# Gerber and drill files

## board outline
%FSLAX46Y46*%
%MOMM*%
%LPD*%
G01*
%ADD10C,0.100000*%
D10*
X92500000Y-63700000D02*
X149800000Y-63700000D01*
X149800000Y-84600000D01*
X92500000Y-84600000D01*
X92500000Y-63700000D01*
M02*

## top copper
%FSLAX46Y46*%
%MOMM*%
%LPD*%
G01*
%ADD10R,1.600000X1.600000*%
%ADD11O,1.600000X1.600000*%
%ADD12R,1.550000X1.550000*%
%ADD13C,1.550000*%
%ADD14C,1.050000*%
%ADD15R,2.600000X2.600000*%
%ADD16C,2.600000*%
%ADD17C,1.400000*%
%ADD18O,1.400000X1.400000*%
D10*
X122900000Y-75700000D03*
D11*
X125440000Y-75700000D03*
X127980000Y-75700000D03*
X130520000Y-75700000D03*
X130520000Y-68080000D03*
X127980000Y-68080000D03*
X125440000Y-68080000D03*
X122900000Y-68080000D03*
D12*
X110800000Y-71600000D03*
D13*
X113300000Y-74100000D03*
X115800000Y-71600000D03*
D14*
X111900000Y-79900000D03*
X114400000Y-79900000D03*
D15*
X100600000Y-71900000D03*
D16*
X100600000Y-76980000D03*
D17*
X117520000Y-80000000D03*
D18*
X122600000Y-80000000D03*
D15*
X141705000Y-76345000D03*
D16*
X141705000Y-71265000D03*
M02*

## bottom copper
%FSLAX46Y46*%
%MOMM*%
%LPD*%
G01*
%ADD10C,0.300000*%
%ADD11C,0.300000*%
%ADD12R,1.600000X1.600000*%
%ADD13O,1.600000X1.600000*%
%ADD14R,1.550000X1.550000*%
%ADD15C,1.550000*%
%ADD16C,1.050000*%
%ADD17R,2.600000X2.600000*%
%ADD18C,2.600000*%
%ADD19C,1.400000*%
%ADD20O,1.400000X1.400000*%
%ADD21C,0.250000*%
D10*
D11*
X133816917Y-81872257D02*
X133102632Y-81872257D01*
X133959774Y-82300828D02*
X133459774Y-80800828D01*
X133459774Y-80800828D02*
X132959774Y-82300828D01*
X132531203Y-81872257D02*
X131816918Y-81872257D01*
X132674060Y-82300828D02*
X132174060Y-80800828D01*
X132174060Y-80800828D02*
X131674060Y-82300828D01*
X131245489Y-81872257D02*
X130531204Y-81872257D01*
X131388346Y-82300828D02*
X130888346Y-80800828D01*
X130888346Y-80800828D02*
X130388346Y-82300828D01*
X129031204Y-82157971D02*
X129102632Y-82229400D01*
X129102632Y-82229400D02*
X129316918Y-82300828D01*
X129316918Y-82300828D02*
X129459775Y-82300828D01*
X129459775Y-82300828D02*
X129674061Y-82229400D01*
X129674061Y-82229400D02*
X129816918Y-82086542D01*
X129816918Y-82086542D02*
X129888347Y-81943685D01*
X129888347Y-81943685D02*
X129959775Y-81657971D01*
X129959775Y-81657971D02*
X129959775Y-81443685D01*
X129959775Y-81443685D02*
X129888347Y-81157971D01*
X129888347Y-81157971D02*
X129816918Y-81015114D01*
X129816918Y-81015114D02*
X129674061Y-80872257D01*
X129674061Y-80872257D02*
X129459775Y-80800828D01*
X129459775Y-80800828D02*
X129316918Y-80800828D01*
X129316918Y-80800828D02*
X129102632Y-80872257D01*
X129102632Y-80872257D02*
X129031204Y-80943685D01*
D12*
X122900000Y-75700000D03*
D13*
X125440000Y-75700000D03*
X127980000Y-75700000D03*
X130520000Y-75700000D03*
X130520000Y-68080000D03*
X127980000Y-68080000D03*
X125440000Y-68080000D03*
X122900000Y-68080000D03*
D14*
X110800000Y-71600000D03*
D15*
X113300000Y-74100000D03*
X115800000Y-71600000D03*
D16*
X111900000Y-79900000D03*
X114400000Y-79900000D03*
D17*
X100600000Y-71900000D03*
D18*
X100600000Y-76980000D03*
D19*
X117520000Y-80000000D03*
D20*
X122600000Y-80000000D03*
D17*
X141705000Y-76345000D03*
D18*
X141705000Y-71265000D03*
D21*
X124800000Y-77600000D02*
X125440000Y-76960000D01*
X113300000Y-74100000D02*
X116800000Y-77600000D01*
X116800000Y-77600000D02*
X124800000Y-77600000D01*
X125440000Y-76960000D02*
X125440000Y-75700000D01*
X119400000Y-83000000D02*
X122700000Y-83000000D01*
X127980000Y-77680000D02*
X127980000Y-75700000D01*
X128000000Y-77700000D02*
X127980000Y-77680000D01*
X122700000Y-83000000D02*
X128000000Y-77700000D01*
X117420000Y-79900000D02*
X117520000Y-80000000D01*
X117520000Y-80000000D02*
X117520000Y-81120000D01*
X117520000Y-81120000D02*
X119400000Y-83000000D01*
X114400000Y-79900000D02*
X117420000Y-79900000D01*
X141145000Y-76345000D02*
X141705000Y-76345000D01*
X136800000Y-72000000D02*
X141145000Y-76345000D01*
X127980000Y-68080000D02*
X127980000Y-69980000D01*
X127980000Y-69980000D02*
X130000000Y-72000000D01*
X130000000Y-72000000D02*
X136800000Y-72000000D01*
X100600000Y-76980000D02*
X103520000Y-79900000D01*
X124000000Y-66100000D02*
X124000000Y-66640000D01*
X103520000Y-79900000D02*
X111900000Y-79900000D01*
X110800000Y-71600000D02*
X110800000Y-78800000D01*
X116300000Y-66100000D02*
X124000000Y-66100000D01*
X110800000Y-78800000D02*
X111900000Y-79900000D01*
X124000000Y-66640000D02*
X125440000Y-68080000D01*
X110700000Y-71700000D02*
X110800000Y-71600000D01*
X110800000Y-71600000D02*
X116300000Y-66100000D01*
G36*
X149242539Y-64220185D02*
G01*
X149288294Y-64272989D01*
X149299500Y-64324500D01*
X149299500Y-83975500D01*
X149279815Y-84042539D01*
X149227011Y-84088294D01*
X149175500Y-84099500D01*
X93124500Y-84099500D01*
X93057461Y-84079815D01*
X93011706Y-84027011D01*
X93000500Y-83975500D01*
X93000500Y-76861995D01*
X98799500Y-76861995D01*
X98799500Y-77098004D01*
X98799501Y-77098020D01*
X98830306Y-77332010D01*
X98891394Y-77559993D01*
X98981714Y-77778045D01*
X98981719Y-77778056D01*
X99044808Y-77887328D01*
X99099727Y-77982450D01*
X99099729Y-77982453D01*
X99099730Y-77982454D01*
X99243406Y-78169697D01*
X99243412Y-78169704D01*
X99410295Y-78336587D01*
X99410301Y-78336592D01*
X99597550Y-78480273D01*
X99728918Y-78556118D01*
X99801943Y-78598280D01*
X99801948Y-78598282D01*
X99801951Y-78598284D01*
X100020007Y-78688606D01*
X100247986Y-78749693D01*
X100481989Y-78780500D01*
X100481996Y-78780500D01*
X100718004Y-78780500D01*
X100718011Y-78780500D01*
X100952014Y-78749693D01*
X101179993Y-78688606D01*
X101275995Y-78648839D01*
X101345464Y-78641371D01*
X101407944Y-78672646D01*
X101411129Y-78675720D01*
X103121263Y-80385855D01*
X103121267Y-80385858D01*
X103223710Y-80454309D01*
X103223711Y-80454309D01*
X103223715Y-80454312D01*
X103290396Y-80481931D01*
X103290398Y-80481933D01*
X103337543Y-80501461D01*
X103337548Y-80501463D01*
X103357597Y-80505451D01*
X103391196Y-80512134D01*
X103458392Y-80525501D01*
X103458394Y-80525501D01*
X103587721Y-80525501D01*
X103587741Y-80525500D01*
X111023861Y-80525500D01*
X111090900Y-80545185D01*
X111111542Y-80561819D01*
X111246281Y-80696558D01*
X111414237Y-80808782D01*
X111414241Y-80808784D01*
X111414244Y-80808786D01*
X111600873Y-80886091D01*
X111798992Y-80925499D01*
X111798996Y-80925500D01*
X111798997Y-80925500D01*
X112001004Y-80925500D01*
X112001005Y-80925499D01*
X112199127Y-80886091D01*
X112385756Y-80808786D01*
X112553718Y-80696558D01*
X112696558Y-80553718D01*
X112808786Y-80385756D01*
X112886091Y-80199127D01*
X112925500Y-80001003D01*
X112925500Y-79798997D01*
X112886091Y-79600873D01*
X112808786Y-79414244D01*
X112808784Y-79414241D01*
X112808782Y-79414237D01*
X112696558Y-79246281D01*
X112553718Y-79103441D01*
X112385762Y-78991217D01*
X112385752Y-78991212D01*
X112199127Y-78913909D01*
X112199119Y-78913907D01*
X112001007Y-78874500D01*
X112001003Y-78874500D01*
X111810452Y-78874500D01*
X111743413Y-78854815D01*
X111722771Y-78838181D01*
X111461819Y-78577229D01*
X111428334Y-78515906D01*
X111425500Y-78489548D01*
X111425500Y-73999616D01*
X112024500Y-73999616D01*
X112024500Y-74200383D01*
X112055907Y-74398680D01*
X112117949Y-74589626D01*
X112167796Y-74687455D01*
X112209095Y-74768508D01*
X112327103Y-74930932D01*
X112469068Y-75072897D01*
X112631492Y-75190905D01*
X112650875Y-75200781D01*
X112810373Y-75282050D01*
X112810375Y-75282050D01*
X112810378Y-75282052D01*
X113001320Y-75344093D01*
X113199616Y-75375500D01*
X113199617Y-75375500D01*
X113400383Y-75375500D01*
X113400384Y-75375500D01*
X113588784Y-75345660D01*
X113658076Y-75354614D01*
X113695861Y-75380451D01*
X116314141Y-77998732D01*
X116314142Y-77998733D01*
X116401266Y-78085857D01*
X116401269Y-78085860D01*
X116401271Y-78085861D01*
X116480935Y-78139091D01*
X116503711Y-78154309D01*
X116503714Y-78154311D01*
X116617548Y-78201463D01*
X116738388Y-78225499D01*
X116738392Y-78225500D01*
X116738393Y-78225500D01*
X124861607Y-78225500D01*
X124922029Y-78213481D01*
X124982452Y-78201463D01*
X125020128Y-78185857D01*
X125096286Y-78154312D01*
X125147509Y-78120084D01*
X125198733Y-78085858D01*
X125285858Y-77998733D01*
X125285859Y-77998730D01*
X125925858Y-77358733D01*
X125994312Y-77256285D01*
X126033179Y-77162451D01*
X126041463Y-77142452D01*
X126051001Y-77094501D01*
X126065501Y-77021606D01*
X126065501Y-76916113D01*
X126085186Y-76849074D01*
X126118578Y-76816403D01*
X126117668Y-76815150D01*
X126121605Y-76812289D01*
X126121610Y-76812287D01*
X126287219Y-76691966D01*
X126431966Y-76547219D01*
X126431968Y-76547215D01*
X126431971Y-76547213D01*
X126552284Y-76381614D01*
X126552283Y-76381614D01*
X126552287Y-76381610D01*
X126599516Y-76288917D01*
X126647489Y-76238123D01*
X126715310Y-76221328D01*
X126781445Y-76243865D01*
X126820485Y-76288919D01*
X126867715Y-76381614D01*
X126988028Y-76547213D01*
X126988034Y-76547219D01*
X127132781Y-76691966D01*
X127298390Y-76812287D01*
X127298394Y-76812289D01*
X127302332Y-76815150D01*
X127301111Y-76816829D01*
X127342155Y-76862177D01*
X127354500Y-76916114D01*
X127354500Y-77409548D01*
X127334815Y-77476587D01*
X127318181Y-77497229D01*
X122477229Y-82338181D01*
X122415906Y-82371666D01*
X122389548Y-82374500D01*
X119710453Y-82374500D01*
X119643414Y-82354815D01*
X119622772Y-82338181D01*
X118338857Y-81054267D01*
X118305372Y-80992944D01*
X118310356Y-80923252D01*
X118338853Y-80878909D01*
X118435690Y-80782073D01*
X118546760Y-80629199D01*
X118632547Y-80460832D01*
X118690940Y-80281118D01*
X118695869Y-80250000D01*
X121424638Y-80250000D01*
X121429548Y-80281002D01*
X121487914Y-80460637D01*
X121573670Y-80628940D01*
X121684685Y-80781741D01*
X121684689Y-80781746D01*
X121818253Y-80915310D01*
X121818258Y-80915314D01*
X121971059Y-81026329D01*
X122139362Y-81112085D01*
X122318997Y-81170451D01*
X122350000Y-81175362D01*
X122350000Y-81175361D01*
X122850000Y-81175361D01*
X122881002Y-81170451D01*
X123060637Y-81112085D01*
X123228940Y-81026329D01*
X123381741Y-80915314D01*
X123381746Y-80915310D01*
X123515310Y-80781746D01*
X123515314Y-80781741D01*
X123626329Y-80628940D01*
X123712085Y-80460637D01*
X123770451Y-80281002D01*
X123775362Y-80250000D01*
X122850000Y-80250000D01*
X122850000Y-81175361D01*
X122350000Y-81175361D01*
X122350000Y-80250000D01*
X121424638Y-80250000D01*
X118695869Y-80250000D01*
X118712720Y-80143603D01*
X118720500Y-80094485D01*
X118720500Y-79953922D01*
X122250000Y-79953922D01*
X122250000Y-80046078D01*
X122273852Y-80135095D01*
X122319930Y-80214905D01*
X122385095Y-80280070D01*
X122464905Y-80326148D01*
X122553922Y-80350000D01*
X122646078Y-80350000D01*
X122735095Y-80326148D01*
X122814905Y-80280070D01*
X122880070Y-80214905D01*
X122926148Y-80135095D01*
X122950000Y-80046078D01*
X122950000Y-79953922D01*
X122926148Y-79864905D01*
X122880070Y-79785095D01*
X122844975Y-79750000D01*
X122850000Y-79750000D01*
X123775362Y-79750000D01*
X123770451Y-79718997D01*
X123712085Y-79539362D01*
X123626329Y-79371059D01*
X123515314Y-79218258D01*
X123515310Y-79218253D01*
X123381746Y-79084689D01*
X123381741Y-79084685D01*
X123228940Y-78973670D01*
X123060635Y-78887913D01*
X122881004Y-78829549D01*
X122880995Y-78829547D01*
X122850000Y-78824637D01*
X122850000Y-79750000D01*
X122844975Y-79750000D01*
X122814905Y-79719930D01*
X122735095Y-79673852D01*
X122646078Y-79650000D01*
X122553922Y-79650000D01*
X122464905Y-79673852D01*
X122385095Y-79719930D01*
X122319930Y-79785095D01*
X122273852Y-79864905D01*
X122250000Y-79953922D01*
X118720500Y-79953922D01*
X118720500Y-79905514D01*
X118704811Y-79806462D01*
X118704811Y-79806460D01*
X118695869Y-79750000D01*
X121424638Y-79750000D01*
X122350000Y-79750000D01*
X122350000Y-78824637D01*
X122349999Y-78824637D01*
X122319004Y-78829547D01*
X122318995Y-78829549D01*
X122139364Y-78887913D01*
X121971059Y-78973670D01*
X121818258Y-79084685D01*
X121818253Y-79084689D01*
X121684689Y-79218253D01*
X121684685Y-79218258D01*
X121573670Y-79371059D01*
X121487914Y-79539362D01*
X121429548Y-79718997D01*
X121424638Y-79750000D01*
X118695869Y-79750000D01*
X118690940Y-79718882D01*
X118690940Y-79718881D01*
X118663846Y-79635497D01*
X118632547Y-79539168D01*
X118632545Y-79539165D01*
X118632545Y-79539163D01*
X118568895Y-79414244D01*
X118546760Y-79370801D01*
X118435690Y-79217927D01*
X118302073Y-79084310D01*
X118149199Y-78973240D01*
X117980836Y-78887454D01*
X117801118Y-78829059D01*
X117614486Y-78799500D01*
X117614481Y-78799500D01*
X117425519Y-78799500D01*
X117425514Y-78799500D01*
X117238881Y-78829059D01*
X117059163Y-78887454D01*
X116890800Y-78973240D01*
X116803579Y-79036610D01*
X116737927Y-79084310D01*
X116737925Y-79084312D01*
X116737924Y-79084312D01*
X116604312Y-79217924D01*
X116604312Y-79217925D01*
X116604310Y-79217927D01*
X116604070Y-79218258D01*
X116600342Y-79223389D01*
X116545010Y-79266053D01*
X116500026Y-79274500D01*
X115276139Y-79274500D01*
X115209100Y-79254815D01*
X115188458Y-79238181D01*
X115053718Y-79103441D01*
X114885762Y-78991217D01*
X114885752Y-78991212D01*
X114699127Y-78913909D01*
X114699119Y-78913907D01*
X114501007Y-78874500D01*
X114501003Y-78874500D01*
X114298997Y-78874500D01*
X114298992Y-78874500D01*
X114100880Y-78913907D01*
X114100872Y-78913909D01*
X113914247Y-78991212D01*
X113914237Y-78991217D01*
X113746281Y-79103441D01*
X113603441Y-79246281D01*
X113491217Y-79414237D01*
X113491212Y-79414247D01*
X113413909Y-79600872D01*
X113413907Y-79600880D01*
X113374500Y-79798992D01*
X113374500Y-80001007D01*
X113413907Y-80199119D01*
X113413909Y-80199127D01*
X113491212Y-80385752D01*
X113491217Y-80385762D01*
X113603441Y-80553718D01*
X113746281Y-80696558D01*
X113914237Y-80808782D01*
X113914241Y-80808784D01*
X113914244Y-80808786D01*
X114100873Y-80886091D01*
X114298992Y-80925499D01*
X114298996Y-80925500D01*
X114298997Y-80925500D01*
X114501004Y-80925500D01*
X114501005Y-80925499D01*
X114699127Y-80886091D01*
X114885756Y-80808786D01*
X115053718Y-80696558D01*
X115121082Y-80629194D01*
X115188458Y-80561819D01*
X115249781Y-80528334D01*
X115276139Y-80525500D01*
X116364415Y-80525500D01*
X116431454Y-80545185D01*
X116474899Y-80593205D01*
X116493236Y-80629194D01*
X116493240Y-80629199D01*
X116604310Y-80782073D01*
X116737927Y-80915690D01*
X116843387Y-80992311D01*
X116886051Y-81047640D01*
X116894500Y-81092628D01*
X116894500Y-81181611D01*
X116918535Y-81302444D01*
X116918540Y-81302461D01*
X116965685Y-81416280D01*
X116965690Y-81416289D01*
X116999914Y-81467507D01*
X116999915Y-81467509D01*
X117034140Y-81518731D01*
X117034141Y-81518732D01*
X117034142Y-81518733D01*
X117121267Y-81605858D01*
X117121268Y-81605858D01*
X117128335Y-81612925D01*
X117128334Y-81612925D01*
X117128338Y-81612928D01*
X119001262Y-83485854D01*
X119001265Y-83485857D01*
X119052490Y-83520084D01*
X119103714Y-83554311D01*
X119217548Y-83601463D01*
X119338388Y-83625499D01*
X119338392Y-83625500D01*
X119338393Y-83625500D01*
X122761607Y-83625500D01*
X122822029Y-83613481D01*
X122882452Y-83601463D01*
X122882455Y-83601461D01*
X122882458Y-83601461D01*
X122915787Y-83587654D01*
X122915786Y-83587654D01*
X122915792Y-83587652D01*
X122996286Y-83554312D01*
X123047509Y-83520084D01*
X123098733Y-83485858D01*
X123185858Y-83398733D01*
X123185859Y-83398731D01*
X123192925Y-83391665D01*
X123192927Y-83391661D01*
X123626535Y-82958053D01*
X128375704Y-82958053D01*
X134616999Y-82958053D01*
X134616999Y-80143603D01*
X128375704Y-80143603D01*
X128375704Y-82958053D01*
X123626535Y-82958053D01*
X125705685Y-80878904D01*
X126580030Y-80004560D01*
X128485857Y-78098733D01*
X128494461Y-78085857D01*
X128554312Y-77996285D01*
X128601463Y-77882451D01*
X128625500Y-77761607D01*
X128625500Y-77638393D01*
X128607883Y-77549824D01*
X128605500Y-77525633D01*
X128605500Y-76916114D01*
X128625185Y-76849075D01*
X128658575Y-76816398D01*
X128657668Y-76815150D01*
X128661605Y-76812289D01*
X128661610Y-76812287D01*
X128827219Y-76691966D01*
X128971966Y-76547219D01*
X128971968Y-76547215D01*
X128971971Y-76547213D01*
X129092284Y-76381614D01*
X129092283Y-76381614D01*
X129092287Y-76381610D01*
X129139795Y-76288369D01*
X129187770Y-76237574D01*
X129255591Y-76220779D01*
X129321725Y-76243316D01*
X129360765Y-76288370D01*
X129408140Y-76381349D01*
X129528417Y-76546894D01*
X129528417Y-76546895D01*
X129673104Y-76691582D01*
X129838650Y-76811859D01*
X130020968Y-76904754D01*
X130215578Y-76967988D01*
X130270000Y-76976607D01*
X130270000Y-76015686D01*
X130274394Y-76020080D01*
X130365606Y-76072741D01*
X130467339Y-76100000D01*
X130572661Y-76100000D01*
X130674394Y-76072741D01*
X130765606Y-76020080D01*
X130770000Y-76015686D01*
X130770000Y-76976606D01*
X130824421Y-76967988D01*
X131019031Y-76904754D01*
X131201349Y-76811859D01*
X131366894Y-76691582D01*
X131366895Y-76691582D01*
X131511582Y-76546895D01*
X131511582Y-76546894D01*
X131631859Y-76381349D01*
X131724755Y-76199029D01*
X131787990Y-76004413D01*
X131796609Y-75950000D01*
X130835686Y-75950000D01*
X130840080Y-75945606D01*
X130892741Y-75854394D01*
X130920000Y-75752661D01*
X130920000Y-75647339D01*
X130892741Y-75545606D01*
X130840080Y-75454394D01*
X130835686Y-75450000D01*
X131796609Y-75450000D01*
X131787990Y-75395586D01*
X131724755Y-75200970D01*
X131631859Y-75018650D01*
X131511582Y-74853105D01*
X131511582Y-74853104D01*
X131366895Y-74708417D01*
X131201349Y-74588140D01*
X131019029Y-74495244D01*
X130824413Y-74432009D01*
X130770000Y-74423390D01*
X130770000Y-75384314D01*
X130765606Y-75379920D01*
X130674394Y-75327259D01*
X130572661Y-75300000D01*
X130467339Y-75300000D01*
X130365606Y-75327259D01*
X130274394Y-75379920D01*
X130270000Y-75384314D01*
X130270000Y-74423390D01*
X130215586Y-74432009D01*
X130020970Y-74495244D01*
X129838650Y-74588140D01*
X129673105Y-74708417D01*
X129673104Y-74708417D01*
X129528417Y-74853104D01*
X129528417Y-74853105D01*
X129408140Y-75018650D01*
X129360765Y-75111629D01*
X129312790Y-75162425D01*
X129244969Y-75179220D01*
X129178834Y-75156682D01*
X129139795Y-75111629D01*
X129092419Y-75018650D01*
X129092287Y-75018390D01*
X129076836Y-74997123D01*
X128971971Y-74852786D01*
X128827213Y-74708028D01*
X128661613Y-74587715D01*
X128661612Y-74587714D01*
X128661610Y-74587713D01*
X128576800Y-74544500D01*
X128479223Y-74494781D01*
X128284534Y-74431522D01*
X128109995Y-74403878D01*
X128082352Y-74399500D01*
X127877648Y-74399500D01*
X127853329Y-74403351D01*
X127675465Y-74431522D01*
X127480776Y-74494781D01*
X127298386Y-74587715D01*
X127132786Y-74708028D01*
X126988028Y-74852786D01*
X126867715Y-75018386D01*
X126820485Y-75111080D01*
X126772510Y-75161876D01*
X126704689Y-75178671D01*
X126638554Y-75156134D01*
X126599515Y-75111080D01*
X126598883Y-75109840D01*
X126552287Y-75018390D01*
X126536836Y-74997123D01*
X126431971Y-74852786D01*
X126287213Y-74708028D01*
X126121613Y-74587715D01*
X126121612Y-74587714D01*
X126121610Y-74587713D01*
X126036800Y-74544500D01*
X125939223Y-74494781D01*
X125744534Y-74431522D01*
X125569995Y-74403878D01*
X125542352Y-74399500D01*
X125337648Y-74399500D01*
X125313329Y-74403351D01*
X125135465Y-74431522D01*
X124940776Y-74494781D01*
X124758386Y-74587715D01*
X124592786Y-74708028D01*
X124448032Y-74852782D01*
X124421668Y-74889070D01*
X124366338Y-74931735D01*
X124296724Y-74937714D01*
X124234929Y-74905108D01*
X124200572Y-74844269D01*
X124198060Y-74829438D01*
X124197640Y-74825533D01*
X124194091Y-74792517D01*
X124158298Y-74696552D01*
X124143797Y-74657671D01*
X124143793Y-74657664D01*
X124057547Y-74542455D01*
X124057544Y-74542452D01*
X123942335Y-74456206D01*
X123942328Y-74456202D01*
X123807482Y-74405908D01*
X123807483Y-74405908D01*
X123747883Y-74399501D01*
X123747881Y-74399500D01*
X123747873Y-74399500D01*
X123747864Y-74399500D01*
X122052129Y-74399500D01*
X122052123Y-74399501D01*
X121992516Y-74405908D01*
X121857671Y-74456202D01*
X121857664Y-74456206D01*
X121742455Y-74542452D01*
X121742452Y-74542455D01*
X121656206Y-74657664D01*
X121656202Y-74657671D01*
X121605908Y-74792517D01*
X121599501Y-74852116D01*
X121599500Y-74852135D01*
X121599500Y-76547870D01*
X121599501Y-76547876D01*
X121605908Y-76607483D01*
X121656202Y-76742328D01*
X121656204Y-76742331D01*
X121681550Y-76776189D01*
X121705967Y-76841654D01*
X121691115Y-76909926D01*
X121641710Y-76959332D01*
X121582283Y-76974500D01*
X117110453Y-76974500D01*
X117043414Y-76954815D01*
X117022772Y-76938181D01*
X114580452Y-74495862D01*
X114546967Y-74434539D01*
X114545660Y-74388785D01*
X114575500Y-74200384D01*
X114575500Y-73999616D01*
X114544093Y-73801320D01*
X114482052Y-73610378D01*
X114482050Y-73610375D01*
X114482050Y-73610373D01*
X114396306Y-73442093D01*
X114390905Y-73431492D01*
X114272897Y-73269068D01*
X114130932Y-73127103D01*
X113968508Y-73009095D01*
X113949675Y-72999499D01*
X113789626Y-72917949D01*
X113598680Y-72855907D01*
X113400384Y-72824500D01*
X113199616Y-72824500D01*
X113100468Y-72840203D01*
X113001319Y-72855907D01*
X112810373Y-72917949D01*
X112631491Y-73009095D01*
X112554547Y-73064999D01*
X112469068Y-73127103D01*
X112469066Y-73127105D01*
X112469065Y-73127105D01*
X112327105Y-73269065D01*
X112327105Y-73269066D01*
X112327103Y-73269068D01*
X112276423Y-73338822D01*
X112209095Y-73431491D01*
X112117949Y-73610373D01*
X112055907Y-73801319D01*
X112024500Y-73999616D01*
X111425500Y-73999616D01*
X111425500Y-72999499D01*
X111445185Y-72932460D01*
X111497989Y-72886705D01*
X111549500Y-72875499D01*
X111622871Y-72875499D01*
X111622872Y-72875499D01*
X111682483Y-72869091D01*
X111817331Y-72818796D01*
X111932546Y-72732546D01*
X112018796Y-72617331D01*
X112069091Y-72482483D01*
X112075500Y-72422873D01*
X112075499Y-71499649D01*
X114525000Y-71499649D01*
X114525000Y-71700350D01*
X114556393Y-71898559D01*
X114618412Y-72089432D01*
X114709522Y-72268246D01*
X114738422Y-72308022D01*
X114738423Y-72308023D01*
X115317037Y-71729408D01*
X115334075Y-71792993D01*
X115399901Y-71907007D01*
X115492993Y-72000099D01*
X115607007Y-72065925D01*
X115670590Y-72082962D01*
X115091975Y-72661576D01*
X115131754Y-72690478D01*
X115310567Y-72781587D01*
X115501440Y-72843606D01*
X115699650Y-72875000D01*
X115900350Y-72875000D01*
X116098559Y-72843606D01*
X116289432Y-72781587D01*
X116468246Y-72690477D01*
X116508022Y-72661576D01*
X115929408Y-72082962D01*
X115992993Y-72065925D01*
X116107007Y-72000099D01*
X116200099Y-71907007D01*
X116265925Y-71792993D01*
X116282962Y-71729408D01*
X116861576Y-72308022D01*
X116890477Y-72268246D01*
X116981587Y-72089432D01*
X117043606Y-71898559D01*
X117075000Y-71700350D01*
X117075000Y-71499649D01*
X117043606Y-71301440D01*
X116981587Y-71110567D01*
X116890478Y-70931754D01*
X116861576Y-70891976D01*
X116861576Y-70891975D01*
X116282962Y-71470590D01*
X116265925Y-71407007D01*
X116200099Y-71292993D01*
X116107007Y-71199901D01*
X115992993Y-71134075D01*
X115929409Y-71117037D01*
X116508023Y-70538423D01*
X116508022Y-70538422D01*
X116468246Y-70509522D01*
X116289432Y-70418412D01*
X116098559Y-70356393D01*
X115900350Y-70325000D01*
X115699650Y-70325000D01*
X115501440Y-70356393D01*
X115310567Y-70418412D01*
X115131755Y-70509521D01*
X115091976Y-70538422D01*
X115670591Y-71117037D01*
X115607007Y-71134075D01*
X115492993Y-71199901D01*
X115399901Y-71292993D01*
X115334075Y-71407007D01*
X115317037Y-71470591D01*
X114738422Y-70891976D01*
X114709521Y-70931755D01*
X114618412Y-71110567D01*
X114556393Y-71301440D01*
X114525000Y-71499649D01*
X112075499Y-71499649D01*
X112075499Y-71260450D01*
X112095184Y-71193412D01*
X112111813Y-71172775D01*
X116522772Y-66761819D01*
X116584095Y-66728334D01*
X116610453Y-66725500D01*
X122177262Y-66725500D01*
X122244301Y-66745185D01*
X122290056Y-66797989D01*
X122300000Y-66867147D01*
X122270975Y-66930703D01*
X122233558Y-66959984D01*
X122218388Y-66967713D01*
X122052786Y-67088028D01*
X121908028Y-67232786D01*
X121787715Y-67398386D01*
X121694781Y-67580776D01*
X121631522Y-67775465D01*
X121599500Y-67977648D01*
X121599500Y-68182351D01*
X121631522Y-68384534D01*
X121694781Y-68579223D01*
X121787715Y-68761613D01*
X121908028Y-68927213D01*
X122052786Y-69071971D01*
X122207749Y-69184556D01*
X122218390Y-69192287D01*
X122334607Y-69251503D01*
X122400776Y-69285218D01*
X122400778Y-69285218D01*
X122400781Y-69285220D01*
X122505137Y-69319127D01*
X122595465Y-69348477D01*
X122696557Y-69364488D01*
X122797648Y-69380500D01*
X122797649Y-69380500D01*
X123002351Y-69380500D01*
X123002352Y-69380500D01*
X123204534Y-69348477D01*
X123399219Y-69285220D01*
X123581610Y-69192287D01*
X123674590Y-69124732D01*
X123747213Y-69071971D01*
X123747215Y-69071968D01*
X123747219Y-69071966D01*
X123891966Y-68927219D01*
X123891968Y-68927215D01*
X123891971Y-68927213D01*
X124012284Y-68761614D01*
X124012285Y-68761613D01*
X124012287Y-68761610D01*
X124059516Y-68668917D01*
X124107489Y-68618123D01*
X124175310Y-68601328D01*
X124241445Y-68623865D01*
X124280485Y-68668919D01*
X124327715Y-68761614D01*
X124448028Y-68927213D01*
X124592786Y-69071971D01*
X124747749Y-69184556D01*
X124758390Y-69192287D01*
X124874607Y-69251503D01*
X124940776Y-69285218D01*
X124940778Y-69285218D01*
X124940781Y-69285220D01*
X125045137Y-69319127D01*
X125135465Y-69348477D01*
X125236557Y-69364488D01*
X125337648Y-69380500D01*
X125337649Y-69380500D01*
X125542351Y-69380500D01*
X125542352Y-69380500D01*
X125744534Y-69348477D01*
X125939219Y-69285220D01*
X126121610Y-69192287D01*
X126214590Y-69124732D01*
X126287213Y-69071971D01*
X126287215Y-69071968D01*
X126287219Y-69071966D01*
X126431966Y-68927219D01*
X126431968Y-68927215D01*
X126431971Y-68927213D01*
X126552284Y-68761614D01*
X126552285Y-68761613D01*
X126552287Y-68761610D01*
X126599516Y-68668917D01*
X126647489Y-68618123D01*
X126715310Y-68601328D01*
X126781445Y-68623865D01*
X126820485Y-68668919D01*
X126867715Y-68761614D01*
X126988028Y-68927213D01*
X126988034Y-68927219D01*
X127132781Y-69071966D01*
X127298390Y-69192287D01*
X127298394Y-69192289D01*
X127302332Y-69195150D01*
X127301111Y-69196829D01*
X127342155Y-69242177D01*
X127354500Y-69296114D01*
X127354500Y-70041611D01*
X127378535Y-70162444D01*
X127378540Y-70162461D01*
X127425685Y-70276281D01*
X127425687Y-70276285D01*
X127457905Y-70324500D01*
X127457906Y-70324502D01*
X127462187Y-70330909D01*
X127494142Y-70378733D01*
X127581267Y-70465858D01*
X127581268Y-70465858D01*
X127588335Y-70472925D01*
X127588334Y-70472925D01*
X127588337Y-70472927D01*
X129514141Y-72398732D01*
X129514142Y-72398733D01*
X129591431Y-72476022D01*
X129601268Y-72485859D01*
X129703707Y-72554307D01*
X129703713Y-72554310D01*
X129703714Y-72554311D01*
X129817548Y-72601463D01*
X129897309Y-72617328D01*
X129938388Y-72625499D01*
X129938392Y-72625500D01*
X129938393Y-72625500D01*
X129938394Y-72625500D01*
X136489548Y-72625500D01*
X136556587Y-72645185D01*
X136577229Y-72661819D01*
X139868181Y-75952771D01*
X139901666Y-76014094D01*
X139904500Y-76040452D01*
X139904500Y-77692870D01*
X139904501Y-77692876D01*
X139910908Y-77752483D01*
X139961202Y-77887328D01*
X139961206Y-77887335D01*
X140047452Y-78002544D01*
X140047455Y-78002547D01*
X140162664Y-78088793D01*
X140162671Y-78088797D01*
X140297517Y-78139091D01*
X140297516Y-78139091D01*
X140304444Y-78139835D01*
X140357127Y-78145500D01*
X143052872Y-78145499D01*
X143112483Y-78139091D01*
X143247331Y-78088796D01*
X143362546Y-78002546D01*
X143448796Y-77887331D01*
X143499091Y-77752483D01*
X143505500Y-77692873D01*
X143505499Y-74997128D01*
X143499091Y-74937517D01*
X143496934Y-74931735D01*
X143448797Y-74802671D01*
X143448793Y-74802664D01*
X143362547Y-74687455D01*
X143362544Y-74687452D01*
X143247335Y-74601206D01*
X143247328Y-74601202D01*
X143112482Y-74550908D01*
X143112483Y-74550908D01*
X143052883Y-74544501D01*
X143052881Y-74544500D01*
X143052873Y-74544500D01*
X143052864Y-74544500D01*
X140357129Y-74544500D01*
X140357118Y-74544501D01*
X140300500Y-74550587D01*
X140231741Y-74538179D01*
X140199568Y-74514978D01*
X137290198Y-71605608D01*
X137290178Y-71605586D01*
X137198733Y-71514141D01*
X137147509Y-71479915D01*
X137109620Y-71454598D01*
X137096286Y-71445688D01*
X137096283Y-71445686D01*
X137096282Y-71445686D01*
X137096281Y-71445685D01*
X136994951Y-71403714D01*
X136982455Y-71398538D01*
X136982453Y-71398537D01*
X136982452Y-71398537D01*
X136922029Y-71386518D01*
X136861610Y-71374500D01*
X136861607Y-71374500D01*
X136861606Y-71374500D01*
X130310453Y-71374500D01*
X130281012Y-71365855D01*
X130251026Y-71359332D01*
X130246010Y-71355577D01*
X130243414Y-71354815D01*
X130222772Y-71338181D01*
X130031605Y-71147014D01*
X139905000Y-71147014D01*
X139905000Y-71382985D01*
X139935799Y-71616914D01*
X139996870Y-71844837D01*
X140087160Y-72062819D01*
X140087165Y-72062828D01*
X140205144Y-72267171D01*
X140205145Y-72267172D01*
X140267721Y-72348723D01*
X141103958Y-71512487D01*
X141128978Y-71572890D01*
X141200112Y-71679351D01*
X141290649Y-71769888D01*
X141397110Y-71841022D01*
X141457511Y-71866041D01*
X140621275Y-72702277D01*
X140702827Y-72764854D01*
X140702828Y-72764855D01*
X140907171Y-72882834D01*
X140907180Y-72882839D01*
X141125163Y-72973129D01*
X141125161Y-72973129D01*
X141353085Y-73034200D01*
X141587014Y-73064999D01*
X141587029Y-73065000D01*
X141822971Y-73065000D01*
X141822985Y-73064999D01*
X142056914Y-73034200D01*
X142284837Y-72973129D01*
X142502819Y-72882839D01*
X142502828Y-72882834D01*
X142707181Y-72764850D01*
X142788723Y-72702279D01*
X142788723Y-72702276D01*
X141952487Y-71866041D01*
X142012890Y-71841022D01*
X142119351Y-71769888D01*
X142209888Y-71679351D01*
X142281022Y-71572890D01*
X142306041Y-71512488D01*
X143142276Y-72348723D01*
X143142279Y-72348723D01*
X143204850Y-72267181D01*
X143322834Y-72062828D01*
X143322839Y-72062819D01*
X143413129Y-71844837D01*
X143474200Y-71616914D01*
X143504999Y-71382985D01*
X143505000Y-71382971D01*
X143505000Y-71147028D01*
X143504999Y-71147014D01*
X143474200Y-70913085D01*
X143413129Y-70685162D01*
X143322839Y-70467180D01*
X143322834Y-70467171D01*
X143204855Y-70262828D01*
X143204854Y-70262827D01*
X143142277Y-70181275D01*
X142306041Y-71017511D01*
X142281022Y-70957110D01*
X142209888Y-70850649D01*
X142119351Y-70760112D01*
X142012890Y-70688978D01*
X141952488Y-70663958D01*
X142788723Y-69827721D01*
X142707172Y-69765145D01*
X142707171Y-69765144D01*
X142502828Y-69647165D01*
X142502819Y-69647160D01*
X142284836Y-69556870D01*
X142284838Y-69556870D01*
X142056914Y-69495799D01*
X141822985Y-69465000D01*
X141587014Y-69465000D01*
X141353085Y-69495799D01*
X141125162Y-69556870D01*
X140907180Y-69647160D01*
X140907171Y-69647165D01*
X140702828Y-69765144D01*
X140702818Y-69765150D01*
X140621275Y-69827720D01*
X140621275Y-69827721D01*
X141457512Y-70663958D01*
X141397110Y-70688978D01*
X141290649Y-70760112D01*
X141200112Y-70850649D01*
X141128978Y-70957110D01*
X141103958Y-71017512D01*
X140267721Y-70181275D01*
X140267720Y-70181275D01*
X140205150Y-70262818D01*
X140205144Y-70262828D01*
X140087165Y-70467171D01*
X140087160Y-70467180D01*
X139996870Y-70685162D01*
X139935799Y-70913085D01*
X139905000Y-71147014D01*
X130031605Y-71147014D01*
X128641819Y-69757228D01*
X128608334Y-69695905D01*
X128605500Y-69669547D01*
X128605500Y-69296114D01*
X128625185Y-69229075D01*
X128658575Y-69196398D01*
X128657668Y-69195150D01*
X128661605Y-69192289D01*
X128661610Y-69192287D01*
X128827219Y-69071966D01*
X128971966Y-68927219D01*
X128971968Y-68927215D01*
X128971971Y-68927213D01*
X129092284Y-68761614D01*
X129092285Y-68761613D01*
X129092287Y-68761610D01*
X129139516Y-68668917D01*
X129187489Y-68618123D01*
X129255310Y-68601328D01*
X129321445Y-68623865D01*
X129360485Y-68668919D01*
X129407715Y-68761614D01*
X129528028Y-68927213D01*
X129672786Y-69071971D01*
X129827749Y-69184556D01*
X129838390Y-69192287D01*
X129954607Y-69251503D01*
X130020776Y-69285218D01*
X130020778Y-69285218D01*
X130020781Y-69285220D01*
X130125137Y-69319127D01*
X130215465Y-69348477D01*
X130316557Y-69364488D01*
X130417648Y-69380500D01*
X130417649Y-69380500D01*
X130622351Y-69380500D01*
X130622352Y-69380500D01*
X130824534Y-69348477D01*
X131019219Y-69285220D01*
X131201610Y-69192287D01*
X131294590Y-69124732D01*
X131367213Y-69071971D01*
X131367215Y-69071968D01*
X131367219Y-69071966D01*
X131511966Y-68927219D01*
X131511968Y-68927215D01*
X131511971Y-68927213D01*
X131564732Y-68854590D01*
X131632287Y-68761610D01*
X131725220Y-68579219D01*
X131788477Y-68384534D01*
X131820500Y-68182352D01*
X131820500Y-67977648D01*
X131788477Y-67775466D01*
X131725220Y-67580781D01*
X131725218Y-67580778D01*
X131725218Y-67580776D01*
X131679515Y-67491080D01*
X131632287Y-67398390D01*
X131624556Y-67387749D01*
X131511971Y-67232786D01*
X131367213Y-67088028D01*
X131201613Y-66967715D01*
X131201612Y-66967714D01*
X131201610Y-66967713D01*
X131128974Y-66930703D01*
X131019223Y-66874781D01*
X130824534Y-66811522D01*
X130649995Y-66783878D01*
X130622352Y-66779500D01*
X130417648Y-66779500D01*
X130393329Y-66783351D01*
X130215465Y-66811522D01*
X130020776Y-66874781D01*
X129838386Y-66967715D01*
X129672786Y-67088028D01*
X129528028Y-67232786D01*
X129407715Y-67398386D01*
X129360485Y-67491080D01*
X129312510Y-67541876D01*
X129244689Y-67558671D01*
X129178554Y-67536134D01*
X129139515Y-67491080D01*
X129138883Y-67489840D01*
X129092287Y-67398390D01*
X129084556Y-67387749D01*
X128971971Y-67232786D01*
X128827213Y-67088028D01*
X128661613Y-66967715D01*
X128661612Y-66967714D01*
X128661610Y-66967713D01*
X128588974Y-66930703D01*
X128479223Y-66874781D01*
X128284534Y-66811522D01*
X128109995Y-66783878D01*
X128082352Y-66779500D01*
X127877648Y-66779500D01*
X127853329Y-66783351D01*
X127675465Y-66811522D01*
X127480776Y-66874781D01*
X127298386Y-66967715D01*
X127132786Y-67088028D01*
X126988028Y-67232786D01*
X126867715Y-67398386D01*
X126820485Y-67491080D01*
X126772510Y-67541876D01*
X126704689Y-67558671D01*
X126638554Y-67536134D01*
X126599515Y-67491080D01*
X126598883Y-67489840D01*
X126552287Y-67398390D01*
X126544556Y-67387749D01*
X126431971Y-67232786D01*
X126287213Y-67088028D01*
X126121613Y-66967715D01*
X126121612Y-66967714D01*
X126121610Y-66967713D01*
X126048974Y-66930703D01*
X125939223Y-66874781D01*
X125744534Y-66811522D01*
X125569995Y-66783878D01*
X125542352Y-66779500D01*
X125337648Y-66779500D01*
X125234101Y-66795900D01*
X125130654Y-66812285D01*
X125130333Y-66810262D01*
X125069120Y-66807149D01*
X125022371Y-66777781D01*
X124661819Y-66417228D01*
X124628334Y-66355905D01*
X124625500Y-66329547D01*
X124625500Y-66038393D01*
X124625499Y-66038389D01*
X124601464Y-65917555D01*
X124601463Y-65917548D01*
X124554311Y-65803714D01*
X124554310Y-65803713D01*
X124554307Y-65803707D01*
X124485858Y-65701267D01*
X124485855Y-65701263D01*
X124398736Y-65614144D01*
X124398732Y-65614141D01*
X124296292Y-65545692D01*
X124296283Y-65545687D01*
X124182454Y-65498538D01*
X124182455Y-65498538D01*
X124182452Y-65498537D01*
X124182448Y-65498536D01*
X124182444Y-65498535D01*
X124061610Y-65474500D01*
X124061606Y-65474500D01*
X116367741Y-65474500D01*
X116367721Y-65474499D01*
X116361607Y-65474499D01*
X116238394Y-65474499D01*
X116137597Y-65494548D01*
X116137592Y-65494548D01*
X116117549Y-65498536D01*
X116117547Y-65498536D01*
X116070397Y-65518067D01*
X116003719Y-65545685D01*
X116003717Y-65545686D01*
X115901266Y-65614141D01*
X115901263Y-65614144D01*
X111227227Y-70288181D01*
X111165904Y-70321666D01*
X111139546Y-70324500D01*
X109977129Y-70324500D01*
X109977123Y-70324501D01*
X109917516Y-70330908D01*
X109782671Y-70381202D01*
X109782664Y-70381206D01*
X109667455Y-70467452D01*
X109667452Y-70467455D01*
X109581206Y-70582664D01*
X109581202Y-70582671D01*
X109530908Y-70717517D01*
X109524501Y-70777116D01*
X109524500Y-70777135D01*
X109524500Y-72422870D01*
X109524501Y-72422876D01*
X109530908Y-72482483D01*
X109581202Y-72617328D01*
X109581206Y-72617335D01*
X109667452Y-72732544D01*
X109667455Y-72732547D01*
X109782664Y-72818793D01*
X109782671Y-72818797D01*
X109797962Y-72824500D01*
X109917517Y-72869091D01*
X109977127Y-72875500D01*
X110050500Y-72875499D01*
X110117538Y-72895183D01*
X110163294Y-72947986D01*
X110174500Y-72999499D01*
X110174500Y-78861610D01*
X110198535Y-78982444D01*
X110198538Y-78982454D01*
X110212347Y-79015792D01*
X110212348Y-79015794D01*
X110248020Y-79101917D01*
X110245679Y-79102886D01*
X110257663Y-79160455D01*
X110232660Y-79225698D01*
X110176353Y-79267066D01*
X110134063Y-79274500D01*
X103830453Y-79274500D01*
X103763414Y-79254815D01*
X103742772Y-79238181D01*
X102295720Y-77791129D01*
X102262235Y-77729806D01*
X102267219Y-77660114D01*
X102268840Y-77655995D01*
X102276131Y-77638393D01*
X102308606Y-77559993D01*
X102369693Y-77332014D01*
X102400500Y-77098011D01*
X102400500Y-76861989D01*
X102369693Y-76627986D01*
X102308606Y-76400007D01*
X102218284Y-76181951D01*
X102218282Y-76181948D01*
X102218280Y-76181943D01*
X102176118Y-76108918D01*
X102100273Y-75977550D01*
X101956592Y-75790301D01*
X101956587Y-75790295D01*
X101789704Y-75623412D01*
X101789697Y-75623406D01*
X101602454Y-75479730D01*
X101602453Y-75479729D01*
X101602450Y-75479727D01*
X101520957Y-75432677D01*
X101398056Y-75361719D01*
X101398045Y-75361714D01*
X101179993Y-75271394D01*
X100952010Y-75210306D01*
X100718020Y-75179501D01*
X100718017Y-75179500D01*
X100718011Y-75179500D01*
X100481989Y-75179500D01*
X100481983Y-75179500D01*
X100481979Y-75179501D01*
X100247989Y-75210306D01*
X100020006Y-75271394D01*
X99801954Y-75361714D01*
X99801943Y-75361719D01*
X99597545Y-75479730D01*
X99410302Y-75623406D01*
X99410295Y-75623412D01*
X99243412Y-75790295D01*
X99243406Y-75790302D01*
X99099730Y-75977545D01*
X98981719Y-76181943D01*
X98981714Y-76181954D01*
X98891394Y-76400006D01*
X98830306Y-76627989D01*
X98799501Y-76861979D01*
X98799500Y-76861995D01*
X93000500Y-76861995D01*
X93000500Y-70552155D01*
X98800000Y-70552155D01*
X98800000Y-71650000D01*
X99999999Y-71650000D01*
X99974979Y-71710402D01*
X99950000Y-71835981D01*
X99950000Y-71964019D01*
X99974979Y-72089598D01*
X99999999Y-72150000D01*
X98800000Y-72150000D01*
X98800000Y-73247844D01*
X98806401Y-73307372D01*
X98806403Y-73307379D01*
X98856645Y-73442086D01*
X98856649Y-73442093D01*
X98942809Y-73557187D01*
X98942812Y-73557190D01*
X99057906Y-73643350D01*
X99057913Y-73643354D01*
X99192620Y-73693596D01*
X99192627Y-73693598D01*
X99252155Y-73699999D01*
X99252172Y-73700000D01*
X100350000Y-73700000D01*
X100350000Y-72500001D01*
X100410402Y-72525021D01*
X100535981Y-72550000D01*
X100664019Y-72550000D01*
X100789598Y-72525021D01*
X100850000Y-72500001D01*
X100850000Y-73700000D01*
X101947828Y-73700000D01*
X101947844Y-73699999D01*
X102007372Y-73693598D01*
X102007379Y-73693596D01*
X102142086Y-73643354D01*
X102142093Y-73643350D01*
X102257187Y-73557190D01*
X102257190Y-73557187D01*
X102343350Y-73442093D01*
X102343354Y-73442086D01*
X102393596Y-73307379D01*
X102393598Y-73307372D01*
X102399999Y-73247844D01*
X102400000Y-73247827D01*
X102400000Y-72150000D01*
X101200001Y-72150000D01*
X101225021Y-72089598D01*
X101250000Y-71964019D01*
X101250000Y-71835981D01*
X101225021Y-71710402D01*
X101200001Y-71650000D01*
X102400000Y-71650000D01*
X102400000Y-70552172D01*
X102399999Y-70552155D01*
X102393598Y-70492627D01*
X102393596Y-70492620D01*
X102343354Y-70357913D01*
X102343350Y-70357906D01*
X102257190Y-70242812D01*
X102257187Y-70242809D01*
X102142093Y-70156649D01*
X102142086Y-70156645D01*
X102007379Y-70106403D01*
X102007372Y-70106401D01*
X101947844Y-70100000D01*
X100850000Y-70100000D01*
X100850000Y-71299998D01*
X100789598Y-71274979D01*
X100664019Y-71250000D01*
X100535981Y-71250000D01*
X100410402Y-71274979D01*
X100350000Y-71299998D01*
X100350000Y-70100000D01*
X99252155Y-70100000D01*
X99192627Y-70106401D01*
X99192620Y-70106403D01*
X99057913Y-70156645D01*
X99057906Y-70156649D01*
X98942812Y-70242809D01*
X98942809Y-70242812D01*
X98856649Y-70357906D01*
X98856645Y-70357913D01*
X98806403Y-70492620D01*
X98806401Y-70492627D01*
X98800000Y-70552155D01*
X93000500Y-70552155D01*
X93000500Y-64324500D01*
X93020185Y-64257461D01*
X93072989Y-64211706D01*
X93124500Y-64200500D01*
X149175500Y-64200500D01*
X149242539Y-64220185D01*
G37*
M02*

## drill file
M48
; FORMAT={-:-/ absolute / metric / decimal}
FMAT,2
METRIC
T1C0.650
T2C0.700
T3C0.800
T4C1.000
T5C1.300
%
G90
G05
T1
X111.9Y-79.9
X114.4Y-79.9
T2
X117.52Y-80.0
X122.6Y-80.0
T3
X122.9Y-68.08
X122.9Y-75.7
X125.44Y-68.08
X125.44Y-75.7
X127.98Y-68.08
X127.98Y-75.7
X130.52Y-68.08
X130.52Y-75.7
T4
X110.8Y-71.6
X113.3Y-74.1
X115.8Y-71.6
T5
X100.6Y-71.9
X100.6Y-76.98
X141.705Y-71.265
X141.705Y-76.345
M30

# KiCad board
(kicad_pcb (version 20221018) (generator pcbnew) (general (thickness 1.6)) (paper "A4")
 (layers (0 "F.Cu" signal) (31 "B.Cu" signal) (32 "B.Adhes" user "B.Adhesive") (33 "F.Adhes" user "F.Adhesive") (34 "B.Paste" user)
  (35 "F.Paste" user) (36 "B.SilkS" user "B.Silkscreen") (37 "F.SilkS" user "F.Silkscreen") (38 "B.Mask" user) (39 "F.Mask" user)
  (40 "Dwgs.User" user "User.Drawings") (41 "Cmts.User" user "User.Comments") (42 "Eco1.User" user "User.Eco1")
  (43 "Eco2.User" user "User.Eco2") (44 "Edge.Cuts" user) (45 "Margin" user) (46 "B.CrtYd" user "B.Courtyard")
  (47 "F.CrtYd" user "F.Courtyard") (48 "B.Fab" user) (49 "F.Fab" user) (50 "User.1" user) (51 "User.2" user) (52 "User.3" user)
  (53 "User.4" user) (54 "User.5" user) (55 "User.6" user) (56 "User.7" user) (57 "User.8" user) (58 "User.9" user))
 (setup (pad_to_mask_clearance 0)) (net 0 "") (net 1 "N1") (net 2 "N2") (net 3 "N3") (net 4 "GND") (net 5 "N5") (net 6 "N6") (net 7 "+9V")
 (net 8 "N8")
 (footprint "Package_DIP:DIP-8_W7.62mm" (layer "F.Cu") (at 122.9 75.7 90)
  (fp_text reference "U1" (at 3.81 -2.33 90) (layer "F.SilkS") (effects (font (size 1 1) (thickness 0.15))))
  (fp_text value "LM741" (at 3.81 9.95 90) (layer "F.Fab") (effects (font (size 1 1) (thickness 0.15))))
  (pad "1" thru_hole rect (at 0 0 90) (size 1.6 1.6) (drill 0.8) (layers "*.Cu" "*.Mask") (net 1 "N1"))
  (pad "2" thru_hole oval (at 0 2.54 90) (size 1.6 1.6) (drill 0.8) (layers "*.Cu" "*.Mask") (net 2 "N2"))
  (pad "3" thru_hole oval (at 0 5.08 90) (size 1.6 1.6) (drill 0.8) (layers "*.Cu" "*.Mask") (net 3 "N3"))
  (pad "4" thru_hole oval (at 0 7.62 90) (size 1.6 1.6) (drill 0.8) (layers "*.Cu" "*.Mask") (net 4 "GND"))
  (pad "5" thru_hole oval (at 7.62 7.62 90) (size 1.6 1.6) (drill 0.8) (layers "*.Cu" "*.Mask") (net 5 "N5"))
  (pad "6" thru_hole oval (at 7.62 5.08 90) (size 1.6 1.6) (drill 0.8) (layers "*.Cu" "*.Mask") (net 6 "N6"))
  (pad "7" thru_hole oval (at 7.62 2.54 90) (size 1.6 1.6) (drill 0.8) (layers "*.Cu" "*.Mask") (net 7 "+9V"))
  (pad "8" thru_hole oval (at 7.62 0 90) (size 1.6 1.6) (drill 0.8) (layers "*.Cu" "*.Mask") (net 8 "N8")))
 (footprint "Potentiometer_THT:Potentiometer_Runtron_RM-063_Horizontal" (layer "F.Cu") (at 110.8 71.6)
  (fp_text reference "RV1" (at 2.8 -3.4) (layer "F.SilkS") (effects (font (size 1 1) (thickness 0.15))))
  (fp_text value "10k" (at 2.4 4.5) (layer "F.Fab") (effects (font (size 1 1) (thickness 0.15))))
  (pad "1" thru_hole rect (at 0 0) (size 1.55 1.55) (drill 1) (layers "*.Cu" "*.Mask") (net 7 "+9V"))
  (pad "2" thru_hole circle (at 2.5 2.5) (size 1.55 1.55) (drill 1) (layers "*.Cu" "*.Mask") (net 2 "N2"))
  (pad "3" thru_hole circle (at 5 0) (size 1.55 1.55) (drill 1) (layers "*.Cu" "*.Mask") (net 4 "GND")))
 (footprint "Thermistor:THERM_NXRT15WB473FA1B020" (layer "F.Cu") (at 113.15 79.9)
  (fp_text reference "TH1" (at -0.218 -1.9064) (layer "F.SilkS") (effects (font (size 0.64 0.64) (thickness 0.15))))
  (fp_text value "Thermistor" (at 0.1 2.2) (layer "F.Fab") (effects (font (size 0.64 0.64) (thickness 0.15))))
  (pad "1" thru_hole circle (at -1.25 0) (size 1.05 1.05) (drill 0.65) (layers "*.Cu" "*.Mask") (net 7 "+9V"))
  (pad "2" thru_hole circle (at 1.25 0) (size 1.05 1.05) (drill 0.65) (layers "*.Cu" "*.Mask") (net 3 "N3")))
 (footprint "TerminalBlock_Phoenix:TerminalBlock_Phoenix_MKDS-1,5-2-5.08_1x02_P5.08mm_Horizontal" (layer "F.Cu") (at 100.6 71.9 -90)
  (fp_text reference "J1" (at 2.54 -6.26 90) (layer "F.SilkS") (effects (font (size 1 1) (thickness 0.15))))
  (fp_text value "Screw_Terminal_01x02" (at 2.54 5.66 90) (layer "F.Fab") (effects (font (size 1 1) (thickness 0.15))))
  (pad "1" thru_hole rect (at 0 0 270) (size 2.6 2.6) (drill 1.3) (layers "*.Cu" "*.Mask") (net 4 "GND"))
  (pad "2" thru_hole circle (at 5.08 0 270) (size 2.6 2.6) (drill 1.3) (layers "*.Cu" "*.Mask") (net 7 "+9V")))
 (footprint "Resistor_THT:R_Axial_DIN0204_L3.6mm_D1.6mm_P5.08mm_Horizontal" (layer "F.Cu") (at 117.52 80)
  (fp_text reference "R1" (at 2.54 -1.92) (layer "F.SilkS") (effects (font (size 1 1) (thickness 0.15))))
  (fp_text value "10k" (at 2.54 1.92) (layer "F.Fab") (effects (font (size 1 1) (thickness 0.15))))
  (pad "1" thru_hole circle (at 0 0) (size 1.4 1.4) (drill 0.7) (layers "*.Cu" "*.Mask") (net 3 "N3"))
  (pad "2" thru_hole oval (at 5.08 0) (size 1.4 1.4) (drill 0.7) (layers "*.Cu" "*.Mask") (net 4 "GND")))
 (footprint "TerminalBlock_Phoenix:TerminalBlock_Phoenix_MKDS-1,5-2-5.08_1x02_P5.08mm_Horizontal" (layer "F.Cu") (at 141.705 76.345 90)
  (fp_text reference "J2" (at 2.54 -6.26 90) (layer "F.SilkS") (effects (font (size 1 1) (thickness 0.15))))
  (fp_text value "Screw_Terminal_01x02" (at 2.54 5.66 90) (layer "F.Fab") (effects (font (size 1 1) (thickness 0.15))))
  (pad "1" thru_hole rect (at 0 0 90) (size 2.6 2.6) (drill 1.3) (layers "*.Cu" "*.Mask") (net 6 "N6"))
  (pad "2" thru_hole circle (at 5.08 0 90) (size 2.6 2.6) (drill 1.3) (layers "*.Cu" "*.Mask") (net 4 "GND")))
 (gr_rect (start 92.5 63.7) (end 149.8 84.6) (stroke (width 0.1) (type default)) (fill none) (layer "Edge.Cuts"))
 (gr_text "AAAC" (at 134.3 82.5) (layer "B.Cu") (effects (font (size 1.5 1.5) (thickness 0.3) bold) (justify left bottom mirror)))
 (segment (start 124.8 77.6) (end 125.44 76.96) (width 0.25) (layer "B.Cu") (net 2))
 (segment (start 113.3 74.1) (end 116.8 77.6) (width 0.25) (layer "B.Cu") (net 2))
 (segment (start 116.8 77.6) (end 124.8 77.6) (width 0.25) (layer "B.Cu") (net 2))
 (segment (start 125.44 76.96) (end 125.44 75.7) (width 0.25) (layer "B.Cu") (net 2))
 (segment (start 119.4 83) (end 122.7 83) (width 0.25) (layer "B.Cu") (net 3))
 (segment (start 127.98 77.68) (end 127.98 75.7) (width 0.25) (layer "B.Cu") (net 3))
 (segment (start 128 77.7) (end 127.98 77.68) (width 0.25) (layer "B.Cu") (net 3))
 (segment (start 122.7 83) (end 128 77.7) (width 0.25) (layer "B.Cu") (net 3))
 (segment (start 117.42 79.9) (end 117.52 80) (width 0.25) (layer "B.Cu") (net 3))
 (segment (start 117.52 80) (end 117.52 81.12) (width 0.25) (layer "B.Cu") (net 3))
 (segment (start 117.52 81.12) (end 119.4 83) (width 0.25) (layer "B.Cu") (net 3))
 (segment (start 114.4 79.9) (end 117.42 79.9) (width 0.25) (layer "B.Cu") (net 3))
 (segment (start 141.145 76.345) (end 141.705 76.345) (width 0.25) (layer "B.Cu") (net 6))
 (segment (start 136.8 72) (end 141.145 76.345) (width 0.25) (layer "B.Cu") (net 6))
 (segment (start 127.98 68.08) (end 127.98 69.98) (width 0.25) (layer "B.Cu") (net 6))
 (segment (start 127.98 69.98) (end 130 72) (width 0.25) (layer "B.Cu") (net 6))
 (segment (start 130 72) (end 136.8 72) (width 0.25) (layer "B.Cu") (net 6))
 (segment (start 100.6 76.98) (end 103.52 79.9) (width 0.25) (layer "B.Cu") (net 7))
 (segment (start 124 66.1) (end 124 66.64) (width 0.25) (layer "B.Cu") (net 7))
 (segment (start 103.52 79.9) (end 111.9 79.9) (width 0.25) (layer "B.Cu") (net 7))
 (segment (start 110.8 71.6) (end 110.8 78.8) (width 0.25) (layer "B.Cu") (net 7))
 (segment (start 116.3 66.1) (end 124 66.1) (width 0.25) (layer "B.Cu") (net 7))
 (segment (start 110.8 78.8) (end 111.9 79.9) (width 0.25) (layer "B.Cu") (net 7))
 (segment (start 124 66.64) (end 125.44 68.08) (width 0.25) (layer "B.Cu") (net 7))
 (segment (start 110.7 71.7) (end 110.8 71.6) (width 0.25) (layer "B.Cu") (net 7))
 (segment (start 110.8 71.6) (end 116.3 66.1) (width 0.25) (layer "B.Cu") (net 7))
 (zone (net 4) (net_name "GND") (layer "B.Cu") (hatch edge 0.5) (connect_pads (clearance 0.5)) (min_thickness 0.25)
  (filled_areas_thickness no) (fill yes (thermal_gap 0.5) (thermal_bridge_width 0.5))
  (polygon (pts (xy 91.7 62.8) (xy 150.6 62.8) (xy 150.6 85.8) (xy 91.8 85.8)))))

